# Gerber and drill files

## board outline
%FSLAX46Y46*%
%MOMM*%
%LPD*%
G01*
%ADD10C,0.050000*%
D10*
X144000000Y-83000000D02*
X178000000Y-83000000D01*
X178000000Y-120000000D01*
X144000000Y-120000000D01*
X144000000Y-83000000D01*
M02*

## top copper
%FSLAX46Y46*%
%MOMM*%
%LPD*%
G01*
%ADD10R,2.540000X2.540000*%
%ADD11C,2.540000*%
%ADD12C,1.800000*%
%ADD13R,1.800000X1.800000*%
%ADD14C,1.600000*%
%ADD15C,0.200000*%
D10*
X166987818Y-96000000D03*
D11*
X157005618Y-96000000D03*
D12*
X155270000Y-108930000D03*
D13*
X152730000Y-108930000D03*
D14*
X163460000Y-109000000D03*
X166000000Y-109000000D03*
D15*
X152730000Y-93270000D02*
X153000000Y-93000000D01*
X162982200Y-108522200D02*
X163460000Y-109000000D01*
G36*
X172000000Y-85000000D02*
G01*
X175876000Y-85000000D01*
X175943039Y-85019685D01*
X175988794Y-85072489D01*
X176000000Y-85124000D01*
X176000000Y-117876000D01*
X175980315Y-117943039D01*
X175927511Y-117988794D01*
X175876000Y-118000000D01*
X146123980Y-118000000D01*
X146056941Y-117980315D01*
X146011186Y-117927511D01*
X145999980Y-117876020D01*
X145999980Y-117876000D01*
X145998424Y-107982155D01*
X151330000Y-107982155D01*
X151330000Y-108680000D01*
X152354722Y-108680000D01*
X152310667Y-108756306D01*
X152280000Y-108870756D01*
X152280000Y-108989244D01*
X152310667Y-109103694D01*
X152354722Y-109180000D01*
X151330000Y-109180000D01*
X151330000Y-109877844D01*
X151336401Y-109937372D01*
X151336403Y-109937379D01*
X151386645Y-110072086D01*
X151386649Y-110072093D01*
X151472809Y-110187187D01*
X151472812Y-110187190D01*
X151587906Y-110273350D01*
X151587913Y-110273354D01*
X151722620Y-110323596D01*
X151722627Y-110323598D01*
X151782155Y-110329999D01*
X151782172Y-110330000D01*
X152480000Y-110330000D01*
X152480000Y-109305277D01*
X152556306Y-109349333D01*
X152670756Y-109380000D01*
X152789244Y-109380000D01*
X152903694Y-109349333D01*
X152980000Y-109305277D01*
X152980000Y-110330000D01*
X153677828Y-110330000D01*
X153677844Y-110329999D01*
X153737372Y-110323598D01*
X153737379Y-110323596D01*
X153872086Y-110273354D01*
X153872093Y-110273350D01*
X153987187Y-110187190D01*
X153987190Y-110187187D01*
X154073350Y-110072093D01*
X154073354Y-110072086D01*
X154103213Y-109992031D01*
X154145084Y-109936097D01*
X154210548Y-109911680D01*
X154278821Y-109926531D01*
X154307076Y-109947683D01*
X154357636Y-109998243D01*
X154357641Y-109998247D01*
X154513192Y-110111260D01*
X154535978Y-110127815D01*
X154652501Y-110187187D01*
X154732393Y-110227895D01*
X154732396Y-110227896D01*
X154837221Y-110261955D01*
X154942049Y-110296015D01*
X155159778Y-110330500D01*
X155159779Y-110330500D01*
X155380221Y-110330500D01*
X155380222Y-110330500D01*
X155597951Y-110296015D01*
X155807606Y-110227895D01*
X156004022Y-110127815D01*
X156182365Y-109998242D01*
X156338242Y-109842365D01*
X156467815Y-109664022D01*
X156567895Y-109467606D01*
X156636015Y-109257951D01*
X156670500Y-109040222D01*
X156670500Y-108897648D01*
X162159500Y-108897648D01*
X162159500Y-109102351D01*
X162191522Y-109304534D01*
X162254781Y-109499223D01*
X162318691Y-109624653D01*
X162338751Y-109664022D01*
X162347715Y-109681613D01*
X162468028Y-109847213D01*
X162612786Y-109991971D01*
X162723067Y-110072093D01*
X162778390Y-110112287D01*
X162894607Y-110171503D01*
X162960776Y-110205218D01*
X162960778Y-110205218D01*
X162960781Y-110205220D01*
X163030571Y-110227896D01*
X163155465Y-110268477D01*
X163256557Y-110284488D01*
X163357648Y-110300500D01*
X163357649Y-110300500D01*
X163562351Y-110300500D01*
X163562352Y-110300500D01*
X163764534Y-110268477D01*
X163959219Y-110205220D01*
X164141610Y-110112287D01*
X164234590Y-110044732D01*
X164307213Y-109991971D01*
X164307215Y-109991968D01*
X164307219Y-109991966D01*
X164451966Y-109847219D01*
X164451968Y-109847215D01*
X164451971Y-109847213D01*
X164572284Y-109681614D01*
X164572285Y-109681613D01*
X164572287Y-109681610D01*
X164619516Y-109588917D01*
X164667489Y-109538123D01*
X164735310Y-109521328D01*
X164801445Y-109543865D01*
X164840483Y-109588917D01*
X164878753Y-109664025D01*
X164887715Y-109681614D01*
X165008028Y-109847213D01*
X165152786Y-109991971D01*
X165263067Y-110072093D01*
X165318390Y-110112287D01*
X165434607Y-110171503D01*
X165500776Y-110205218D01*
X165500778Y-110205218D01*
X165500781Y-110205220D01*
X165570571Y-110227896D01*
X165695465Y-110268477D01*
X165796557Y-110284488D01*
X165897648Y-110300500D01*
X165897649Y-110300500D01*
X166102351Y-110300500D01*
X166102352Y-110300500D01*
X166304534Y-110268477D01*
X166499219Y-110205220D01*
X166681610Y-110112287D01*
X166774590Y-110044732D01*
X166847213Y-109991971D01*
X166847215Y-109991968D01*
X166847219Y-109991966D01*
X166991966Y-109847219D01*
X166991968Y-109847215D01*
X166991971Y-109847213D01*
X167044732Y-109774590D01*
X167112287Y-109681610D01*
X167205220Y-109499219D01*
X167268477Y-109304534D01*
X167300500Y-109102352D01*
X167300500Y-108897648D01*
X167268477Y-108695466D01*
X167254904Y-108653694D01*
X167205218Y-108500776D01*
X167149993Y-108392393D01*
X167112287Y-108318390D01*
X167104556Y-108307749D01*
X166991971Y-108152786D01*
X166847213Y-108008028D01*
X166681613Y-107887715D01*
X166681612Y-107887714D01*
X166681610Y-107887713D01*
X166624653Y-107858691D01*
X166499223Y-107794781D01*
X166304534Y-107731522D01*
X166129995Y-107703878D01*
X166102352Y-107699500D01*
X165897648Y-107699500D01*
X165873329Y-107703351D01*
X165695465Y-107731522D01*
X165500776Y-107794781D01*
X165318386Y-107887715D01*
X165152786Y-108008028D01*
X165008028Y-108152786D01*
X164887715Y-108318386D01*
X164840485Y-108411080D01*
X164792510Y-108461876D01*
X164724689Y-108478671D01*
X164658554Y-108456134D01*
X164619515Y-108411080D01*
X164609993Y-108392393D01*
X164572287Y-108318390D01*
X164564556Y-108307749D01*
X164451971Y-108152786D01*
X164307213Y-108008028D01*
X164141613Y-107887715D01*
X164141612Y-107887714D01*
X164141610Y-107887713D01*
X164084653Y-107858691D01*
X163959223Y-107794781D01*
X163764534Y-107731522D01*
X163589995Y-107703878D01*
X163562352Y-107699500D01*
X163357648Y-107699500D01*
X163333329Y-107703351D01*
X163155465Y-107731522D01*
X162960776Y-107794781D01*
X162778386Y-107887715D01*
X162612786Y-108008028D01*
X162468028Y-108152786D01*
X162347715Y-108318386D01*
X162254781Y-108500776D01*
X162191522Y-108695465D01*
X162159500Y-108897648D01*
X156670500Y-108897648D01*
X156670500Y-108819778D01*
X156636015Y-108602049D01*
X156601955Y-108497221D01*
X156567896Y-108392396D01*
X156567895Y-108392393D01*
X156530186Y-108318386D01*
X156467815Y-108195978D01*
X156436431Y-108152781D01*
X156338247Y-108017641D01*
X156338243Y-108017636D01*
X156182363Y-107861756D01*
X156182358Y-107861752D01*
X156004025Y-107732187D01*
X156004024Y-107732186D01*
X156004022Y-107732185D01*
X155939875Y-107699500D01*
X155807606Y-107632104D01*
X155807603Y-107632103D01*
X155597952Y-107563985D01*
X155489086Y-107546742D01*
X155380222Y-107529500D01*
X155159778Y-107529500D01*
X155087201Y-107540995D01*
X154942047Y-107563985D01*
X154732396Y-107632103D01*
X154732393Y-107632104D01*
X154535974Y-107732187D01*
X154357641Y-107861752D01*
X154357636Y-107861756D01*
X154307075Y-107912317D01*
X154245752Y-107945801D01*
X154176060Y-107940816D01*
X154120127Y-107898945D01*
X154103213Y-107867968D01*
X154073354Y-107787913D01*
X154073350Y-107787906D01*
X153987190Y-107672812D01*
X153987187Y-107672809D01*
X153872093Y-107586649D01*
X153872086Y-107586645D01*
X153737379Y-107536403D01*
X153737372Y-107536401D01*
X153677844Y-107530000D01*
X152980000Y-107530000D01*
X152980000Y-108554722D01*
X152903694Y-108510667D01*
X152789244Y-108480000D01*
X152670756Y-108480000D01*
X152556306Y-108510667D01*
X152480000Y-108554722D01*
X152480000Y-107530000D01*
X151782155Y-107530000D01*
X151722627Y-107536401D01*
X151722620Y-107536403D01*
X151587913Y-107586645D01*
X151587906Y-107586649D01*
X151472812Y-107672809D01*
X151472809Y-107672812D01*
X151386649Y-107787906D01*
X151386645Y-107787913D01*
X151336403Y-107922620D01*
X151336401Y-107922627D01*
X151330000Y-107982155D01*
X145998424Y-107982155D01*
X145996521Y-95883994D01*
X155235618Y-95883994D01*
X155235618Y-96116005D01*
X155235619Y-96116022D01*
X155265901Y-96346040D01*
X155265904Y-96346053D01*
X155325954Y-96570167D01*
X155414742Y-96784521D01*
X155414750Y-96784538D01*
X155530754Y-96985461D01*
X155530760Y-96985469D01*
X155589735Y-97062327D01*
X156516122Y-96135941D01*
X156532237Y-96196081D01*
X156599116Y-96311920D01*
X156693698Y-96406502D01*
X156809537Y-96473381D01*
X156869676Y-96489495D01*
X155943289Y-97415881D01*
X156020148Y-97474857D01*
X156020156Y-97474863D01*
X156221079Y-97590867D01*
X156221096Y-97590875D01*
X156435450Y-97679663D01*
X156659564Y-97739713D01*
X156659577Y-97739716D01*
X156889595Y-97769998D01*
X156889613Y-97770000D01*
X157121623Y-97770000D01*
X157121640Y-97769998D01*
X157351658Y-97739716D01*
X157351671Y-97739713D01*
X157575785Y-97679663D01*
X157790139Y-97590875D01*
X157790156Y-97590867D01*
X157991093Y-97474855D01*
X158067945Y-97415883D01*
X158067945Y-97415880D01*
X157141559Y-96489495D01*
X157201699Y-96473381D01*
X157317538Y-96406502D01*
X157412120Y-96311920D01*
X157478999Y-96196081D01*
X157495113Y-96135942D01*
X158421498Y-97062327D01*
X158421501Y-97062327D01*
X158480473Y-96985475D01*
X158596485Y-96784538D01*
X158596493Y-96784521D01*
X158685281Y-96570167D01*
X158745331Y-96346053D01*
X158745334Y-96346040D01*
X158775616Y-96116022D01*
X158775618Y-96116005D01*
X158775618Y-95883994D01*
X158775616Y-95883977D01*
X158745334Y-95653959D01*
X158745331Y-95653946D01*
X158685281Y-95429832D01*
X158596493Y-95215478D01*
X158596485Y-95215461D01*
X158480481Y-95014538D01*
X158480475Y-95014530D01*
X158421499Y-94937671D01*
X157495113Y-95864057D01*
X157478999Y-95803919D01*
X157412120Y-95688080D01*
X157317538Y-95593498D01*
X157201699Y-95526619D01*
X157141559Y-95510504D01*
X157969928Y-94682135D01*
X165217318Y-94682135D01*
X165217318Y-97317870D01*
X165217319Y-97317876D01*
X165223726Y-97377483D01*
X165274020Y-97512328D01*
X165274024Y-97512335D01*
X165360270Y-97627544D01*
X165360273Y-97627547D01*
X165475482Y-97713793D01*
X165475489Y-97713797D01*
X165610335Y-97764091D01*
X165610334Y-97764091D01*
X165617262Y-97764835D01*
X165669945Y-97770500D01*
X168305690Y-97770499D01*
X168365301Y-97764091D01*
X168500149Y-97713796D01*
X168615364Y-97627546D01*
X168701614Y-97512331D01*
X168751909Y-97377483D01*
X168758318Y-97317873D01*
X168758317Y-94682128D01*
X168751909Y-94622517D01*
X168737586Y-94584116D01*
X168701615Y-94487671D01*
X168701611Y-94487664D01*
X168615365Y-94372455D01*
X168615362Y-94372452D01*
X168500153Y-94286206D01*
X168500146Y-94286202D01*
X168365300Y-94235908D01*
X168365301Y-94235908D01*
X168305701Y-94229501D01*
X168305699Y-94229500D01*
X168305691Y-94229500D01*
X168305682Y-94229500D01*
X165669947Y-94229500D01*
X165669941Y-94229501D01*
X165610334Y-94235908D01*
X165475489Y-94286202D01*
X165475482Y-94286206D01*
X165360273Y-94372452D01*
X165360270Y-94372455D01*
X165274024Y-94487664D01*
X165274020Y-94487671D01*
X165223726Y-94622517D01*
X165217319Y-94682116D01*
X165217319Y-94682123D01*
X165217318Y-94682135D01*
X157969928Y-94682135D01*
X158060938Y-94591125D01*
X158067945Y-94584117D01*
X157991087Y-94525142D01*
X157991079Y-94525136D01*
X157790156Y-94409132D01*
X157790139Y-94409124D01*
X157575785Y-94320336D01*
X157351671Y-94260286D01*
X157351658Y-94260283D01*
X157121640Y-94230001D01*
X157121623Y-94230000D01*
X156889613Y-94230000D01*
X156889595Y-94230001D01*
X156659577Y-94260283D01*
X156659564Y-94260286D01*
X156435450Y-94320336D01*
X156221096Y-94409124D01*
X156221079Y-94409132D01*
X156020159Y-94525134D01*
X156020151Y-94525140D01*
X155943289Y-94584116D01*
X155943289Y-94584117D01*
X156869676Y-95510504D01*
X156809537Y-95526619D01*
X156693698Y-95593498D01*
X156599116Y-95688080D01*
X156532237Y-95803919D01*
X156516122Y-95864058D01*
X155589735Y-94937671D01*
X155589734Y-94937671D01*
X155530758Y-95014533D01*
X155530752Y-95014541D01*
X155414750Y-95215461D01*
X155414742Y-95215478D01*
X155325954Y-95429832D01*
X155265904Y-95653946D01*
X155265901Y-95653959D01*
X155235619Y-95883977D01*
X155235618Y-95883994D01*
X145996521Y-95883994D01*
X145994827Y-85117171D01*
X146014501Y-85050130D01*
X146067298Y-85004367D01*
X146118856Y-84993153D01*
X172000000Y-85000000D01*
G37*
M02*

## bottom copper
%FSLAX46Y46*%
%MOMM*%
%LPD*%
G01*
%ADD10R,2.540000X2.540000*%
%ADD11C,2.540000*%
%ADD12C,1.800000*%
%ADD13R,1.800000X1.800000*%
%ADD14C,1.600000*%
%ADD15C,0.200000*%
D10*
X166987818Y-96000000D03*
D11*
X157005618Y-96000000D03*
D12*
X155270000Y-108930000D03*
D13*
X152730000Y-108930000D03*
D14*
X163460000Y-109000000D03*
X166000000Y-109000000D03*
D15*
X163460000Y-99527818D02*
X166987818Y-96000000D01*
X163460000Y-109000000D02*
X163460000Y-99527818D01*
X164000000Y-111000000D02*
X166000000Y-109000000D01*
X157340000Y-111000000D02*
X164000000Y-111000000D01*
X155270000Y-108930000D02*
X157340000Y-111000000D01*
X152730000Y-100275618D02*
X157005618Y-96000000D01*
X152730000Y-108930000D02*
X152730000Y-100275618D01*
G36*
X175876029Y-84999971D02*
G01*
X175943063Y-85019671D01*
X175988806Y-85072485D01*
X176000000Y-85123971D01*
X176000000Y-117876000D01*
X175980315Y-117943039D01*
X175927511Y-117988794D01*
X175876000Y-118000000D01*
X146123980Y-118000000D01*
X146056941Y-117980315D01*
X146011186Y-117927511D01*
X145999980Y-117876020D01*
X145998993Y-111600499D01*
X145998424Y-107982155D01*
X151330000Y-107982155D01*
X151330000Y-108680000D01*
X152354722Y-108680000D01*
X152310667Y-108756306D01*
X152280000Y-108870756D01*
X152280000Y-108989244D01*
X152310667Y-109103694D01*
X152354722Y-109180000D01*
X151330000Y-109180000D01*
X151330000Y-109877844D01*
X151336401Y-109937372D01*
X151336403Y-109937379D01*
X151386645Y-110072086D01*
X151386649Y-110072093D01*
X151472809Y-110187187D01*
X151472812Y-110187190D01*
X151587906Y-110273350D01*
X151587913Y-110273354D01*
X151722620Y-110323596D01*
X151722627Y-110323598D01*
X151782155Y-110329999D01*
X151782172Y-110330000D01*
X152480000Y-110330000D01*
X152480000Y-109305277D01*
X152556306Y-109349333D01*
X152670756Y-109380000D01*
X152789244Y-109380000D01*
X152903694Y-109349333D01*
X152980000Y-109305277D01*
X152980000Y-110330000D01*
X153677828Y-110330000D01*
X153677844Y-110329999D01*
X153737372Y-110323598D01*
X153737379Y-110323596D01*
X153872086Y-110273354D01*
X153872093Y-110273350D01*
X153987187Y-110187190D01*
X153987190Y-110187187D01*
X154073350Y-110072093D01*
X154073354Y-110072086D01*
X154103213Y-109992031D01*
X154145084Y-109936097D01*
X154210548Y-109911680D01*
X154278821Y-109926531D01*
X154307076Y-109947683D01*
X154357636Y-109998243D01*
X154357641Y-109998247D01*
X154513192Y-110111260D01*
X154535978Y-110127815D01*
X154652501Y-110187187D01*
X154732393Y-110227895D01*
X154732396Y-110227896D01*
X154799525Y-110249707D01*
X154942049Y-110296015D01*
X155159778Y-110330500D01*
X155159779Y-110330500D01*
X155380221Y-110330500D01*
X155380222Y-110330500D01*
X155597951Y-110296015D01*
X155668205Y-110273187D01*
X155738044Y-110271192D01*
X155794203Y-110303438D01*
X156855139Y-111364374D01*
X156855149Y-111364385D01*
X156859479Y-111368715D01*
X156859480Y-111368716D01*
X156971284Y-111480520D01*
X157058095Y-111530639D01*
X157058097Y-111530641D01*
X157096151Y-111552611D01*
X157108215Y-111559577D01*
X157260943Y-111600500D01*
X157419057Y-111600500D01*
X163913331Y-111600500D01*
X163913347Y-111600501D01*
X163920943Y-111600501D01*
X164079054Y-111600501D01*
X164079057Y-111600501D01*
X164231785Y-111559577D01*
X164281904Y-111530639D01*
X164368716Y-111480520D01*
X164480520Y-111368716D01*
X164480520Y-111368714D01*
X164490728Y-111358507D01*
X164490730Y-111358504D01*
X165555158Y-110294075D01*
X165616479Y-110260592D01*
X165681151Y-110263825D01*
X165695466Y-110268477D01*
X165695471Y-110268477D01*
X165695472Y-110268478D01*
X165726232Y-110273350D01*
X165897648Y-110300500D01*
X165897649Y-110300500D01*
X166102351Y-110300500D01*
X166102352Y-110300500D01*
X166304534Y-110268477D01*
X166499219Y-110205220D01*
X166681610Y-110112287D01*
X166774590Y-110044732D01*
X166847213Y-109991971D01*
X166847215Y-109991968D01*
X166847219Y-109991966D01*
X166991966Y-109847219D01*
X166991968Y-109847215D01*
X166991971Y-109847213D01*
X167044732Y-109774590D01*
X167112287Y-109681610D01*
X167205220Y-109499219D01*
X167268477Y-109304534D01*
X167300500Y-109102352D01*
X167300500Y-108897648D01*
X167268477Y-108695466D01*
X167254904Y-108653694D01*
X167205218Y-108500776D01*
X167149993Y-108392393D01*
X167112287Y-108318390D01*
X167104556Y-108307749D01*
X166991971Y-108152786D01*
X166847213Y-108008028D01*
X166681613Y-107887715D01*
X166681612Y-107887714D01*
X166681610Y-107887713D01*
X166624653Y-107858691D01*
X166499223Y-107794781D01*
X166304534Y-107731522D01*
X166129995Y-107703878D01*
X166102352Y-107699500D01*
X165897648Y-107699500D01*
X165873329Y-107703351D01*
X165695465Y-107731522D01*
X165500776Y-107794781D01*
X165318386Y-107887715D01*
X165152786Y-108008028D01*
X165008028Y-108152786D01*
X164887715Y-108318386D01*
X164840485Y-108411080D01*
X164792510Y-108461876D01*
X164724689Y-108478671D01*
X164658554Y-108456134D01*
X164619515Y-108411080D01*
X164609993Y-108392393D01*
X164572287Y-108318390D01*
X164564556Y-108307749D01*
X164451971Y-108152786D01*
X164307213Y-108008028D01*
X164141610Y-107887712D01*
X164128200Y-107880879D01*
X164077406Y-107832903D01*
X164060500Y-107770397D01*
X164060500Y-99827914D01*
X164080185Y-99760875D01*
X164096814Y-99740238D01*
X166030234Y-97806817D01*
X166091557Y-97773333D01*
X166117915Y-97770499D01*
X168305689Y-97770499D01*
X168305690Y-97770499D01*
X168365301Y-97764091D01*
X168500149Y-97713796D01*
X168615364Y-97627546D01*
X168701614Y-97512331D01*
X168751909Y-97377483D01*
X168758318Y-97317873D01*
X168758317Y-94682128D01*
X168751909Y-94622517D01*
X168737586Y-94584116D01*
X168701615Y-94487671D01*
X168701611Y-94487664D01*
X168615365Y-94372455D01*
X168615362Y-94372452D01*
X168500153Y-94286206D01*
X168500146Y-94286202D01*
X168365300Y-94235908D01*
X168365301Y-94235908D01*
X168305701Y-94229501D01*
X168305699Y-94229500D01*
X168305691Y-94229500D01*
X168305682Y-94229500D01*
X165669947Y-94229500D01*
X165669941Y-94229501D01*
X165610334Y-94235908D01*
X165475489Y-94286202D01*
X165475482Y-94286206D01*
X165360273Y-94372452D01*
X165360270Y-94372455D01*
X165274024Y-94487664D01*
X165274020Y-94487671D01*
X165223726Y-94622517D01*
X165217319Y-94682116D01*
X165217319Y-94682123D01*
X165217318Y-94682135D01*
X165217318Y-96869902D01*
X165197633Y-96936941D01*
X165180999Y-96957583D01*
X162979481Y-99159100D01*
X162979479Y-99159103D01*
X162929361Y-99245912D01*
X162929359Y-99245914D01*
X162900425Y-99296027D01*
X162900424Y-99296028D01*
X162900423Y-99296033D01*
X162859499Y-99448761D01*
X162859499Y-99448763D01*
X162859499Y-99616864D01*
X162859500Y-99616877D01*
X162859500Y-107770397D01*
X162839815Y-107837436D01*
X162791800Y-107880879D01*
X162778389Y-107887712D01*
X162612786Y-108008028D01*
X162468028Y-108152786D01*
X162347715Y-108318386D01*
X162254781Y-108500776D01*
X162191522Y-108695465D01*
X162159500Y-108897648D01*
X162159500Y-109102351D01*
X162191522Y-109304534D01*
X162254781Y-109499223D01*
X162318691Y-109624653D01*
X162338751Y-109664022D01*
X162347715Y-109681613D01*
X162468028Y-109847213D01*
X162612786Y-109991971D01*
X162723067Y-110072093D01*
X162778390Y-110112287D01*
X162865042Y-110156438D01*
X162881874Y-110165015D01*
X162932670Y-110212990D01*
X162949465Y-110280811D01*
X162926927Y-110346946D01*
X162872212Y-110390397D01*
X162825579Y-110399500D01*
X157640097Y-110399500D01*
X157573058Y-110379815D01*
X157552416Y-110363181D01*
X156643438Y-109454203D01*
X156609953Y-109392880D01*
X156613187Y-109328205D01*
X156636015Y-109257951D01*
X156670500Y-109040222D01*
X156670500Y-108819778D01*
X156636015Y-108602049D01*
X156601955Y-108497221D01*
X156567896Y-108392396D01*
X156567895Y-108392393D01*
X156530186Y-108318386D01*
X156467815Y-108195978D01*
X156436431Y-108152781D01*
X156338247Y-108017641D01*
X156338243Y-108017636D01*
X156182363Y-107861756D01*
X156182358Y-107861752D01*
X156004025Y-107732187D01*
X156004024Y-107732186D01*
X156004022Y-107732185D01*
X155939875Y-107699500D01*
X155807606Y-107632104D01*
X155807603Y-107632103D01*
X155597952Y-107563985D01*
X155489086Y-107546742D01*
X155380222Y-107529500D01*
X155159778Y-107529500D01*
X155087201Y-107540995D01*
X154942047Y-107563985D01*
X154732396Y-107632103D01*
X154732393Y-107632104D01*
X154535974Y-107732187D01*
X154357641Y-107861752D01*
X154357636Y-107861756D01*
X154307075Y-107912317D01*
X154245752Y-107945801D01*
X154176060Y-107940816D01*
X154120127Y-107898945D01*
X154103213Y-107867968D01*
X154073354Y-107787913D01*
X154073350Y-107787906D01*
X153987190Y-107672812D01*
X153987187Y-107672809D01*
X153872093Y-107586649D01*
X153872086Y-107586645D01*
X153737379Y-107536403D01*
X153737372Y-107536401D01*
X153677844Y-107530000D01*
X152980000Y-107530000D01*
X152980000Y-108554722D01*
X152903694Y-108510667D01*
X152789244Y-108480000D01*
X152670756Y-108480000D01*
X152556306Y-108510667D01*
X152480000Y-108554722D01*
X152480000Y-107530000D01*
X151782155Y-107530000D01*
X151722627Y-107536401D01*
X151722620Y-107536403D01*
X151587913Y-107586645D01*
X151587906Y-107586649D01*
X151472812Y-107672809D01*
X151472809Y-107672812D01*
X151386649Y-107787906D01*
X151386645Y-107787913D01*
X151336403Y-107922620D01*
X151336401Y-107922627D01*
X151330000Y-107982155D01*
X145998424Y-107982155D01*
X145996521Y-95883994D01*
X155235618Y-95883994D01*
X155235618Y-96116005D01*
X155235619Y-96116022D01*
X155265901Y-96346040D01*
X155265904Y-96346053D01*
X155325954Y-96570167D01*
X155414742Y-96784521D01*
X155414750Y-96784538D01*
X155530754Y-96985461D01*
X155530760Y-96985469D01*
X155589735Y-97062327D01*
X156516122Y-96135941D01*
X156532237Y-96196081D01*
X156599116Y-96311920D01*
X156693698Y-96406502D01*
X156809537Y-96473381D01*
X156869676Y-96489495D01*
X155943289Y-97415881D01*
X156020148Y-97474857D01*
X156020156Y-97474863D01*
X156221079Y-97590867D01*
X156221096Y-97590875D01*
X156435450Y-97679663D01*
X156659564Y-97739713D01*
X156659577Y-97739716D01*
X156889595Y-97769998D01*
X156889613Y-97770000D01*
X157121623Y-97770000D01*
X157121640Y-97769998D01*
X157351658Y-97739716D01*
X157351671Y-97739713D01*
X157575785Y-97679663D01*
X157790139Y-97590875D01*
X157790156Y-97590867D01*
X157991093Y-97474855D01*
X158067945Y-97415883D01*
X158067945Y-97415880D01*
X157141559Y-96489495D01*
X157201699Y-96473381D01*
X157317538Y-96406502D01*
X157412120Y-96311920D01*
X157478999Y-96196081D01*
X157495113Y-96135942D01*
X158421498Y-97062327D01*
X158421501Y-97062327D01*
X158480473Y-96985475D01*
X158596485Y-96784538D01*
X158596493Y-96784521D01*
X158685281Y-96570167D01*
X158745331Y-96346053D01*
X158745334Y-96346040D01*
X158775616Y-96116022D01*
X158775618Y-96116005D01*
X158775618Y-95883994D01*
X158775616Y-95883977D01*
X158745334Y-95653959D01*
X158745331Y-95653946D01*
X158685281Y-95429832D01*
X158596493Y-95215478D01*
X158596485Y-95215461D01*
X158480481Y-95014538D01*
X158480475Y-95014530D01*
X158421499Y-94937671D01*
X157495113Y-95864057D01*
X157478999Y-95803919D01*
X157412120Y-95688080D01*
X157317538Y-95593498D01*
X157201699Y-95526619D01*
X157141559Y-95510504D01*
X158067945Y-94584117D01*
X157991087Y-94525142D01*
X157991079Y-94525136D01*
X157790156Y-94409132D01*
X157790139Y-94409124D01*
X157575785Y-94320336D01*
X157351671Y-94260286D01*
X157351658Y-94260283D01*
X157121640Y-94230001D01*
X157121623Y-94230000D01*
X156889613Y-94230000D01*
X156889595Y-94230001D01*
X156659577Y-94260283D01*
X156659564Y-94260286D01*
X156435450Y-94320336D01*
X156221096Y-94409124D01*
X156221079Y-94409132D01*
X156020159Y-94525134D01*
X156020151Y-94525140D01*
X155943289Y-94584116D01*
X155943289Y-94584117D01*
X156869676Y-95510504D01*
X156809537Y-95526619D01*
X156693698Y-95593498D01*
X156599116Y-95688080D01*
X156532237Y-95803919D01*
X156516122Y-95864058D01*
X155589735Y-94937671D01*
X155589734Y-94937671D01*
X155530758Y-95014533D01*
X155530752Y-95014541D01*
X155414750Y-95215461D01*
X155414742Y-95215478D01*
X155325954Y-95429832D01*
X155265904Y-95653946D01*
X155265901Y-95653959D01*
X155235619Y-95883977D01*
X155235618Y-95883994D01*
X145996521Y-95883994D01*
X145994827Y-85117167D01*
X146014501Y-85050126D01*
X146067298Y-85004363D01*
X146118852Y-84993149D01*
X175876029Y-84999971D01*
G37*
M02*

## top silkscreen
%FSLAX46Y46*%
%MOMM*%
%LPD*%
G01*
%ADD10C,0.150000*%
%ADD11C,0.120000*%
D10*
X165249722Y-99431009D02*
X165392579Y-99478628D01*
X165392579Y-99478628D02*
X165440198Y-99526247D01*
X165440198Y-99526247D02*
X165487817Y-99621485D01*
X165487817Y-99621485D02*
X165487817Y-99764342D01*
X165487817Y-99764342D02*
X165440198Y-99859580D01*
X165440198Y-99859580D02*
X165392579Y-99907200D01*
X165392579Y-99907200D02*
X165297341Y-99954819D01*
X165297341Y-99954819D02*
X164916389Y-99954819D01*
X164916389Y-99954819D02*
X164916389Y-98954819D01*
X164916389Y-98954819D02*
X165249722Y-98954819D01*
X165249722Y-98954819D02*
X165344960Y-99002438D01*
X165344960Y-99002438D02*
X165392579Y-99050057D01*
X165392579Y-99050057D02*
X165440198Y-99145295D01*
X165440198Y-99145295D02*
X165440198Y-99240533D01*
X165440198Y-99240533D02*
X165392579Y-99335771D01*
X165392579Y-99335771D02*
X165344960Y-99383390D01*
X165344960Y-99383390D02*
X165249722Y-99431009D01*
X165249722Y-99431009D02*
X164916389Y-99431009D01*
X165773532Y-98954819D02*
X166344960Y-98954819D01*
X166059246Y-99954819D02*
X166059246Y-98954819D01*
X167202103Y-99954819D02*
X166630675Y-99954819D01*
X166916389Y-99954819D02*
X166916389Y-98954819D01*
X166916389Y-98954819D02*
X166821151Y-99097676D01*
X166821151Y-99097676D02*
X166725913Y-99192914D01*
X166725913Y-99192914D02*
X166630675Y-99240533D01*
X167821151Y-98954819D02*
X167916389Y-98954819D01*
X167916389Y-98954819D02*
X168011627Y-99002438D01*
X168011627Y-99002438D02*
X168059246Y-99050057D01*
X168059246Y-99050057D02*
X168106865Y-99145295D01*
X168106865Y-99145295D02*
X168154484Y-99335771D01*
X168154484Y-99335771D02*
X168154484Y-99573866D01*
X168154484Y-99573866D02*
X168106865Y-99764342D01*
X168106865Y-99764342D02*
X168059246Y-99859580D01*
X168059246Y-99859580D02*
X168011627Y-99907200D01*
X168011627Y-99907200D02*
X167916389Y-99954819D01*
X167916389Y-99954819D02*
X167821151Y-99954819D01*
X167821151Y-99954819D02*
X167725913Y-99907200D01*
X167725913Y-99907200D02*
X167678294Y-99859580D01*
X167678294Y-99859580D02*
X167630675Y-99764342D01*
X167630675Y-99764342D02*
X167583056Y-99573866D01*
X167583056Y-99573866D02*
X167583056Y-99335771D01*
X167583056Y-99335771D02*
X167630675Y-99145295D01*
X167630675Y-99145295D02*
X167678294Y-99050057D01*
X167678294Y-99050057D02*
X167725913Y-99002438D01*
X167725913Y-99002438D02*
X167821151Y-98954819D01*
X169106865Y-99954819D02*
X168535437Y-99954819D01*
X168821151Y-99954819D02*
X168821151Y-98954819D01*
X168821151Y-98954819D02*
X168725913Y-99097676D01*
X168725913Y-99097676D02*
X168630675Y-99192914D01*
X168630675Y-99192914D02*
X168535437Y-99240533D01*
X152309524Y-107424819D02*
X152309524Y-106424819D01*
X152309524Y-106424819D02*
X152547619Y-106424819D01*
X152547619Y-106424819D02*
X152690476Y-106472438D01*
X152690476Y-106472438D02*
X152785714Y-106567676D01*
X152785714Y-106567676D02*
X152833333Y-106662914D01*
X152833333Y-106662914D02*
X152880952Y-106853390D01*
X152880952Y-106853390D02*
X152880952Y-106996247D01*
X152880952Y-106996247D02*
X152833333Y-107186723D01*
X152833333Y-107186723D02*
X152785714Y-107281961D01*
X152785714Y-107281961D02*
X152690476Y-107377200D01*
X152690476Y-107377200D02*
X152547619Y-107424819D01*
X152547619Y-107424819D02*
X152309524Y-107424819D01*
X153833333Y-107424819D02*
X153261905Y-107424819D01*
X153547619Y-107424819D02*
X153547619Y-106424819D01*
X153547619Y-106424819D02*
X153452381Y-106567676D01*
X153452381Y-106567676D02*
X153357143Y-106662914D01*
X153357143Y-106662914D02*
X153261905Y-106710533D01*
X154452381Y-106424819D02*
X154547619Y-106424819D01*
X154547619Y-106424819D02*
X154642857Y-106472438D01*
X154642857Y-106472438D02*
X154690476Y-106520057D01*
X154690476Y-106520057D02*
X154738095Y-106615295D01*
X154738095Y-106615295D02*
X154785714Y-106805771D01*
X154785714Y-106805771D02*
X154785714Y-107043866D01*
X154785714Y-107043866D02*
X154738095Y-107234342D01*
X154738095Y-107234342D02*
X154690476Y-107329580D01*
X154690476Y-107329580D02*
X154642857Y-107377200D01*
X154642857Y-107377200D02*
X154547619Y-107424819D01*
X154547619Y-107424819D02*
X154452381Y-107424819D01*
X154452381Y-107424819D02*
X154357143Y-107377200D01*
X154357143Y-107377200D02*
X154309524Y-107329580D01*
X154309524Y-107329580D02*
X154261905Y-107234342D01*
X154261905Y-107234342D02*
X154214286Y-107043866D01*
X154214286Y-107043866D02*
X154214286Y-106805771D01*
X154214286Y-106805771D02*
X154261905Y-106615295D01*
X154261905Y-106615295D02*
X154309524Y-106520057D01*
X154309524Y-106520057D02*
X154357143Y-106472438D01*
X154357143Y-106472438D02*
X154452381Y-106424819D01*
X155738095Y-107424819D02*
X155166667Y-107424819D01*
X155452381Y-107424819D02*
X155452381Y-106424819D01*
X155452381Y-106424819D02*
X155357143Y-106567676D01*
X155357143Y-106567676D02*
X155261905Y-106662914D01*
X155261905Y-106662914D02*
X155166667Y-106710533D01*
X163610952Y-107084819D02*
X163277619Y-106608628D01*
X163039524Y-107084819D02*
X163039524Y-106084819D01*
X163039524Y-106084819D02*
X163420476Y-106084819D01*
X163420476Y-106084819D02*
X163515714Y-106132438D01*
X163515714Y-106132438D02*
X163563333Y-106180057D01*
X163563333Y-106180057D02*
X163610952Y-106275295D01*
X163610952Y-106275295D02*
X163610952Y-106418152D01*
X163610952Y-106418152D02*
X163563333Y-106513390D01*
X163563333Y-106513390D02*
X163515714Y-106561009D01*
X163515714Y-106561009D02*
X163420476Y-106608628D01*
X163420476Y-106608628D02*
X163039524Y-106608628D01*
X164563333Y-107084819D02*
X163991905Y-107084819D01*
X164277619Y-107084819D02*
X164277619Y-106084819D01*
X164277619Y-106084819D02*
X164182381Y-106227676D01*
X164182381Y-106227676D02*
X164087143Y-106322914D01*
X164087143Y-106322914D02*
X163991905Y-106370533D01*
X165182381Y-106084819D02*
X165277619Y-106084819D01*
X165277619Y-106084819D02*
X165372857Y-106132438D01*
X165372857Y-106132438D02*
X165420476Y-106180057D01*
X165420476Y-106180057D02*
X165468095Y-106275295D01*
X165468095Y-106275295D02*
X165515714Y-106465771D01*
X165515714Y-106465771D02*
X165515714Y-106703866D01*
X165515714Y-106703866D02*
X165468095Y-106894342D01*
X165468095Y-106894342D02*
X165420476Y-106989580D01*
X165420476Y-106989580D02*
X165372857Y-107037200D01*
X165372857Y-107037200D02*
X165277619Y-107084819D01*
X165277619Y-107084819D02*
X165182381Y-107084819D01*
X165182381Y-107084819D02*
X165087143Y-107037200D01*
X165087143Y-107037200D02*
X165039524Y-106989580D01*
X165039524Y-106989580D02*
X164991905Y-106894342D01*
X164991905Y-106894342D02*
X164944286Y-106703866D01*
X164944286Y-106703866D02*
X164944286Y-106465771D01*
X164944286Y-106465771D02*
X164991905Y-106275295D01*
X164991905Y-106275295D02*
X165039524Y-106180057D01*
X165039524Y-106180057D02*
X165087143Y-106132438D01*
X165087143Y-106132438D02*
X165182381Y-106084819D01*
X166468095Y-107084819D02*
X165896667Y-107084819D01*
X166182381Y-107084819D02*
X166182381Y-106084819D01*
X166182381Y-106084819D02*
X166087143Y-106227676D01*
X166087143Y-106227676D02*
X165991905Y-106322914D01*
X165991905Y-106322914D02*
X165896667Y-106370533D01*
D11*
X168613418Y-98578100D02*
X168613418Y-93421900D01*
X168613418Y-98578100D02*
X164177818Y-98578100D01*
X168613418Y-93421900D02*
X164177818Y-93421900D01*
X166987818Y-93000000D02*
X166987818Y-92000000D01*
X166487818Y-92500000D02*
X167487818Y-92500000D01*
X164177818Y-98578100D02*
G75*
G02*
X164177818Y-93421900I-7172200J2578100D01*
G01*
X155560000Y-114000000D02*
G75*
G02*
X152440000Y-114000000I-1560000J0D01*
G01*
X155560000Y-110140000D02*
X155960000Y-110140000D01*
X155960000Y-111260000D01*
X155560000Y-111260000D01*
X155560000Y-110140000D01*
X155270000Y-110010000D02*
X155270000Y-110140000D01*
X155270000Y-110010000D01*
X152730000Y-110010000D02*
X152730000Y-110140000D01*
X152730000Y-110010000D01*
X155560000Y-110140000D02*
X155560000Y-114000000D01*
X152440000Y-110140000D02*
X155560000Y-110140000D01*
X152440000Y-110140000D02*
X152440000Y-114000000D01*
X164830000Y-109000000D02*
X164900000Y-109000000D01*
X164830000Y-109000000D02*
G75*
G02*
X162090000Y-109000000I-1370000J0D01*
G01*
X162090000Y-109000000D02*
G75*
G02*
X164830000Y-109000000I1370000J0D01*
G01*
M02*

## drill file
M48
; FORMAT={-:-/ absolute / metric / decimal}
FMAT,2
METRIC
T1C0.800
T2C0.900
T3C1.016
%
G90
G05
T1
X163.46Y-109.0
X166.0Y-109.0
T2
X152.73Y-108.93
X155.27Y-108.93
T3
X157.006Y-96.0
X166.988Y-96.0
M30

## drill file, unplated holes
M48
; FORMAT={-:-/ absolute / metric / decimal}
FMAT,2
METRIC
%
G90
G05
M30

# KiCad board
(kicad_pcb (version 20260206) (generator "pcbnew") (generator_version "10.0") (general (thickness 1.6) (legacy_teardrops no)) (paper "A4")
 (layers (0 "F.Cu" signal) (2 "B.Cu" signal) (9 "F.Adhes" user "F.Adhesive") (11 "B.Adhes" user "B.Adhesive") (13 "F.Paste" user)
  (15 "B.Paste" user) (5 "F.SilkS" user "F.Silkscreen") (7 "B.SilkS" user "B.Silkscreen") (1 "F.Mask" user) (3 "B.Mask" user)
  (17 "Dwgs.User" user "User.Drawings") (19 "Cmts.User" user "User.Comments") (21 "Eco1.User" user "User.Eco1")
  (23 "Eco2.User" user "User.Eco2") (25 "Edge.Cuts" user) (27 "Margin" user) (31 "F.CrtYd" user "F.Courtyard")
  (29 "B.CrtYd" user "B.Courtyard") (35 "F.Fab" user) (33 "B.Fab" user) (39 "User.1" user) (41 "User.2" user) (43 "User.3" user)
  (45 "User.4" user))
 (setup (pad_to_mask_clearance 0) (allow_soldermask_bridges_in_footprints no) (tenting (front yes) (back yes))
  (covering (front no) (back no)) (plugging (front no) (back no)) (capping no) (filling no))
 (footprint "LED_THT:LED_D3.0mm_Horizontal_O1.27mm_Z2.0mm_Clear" (layer "F.Cu") (at 152.73 108.93)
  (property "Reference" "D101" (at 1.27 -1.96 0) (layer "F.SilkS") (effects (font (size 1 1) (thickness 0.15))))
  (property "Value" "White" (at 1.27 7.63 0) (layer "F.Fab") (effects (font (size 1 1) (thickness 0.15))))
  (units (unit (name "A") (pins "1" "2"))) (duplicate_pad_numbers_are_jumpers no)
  (fp_line (start -0.29 1.21) (end -0.29 5.07) (stroke (width 0.12) (type solid)) (layer "F.SilkS"))
  (fp_line (start -0.29 1.21) (end 2.83 1.21) (stroke (width 0.12) (type solid)) (layer "F.SilkS"))
  (fp_line (start 2.83 1.21) (end 2.83 5.07) (stroke (width 0.12) (type solid)) (layer "F.SilkS"))
  (fp_rect (start 0 1.08) (end 0 1.21) (stroke (width 0.12) (type solid)) (fill no) (layer "F.SilkS"))
  (fp_rect (start 2.54 1.08) (end 2.54 1.21) (stroke (width 0.12) (type solid)) (fill no) (layer "F.SilkS"))
  (fp_rect (start 2.83 1.21) (end 3.23 2.33) (stroke (width 0.12) (type solid)) (fill no) (layer "F.SilkS"))
  (fp_arc (start 2.83 5.07) (mid 1.27 6.63) (end -0.29 5.07) (stroke (width 0.12) (type solid)) (layer "F.SilkS"))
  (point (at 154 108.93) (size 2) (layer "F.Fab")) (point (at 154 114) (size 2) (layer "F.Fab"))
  (pad "1" thru_hole rect (at 0 0) (size 1.8 1.8) (drill 0.9) (layers "*.Cu" "*.Mask") (remove_unused_layers no) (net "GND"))
  (pad "2" thru_hole circle (at 2.54 0) (size 1.8 1.8) (drill 0.9) (layers "*.Cu" "*.Mask") (remove_unused_layers no) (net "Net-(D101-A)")))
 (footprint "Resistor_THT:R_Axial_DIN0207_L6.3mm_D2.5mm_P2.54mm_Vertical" (layer "F.Cu") (at 163.46 109)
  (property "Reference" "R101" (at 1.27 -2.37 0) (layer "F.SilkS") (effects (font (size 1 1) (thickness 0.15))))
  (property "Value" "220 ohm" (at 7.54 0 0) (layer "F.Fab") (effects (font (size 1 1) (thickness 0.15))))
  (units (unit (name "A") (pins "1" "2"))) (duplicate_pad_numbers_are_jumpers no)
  (fp_line (start 1.37 0) (end 1.44 0) (stroke (width 0.12) (type solid)) (layer "F.SilkS"))
  (fp_circle (center 0 0) (end 1.37 0) (stroke (width 0.12) (type solid)) (fill no) (layer "F.SilkS"))
  (pad "1" thru_hole circle (at 0 0) (size 1.6 1.6) (drill 0.8) (layers "*.Cu" "*.Mask") (remove_unused_layers no) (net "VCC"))
  (pad "2" thru_hole circle (at 2.54 0) (size 1.6 1.6) (drill 0.8) (layers "*.Cu" "*.Mask") (remove_unused_layers no) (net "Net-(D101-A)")))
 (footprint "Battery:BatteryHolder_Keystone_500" (layer "F.Cu") (at 166.987818 96 180)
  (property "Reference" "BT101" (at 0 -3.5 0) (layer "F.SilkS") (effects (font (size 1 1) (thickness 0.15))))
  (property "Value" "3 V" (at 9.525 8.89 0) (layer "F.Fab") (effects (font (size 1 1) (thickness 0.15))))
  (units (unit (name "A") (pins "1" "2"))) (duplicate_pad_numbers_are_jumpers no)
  (fp_line (start 0.5 3.5) (end -0.5 3.5) (stroke (width 0.12) (type default)) (layer "F.SilkS"))
  (fp_line (start 0 3) (end 0 4) (stroke (width 0.12) (type default)) (layer "F.SilkS"))
  (fp_line (start -1.6256 2.5781) (end 2.81 2.5781) (stroke (width 0.12) (type solid)) (layer "F.SilkS"))
  (fp_line (start -1.6256 -2.5781) (end 2.81 -2.5781) (stroke (width 0.12) (type solid)) (layer "F.SilkS"))
  (fp_line (start -1.6256 -2.5781) (end -1.6256 2.5781) (stroke (width 0.12) (type default)) (layer "F.SilkS"))
  (fp_arc (start 2.81 -2.5781) (mid 17.603686 0) (end 2.81 2.5781) (stroke (width 0.12) (type default)) (layer "F.SilkS"))
  (pad "1" thru_hole rect (at 0 0 180) (size 2.54 2.54) (drill 1.016) (layers "*.Cu" "*.Mask") (remove_unused_layers no) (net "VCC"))
  (pad "2" thru_hole circle (at 9.9822 0 180) (size 2.54 2.54) (drill 1.016) (layers "*.Cu" "*.Mask") (remove_unused_layers no) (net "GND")))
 (gr_rect (start 144 83) (end 178 120) (stroke (width 0.05) (type default)) (fill no) (layer "Edge.Cuts"))
 (segment (start 152.73 93.27) (end 153 93) (width 0.2) (layer "F.Cu") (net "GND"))
 (segment (start 152.73 108.93) (end 152.73 100.275618) (width 0.2) (layer "B.Cu") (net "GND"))
 (segment (start 152.73 100.275618) (end 157.005618 96) (width 0.2) (layer "B.Cu") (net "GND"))
 (segment (start 162.9822 108.5222) (end 163.46 109) (width 0.2) (layer "F.Cu") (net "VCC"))
 (segment (start 163.46 109) (end 163.46 99.527818) (width 0.2) (layer "B.Cu") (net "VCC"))
 (segment (start 163.46 99.527818) (end 166.987818 96) (width 0.2) (layer "B.Cu") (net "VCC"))
 (segment (start 157.34 111) (end 164 111) (width 0.2) (layer "B.Cu") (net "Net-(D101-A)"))
 (segment (start 155.27 108.93) (end 157.34 111) (width 0.2) (layer "B.Cu") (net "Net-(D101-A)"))
 (segment (start 164 111) (end 166 109) (width 0.2) (layer "B.Cu") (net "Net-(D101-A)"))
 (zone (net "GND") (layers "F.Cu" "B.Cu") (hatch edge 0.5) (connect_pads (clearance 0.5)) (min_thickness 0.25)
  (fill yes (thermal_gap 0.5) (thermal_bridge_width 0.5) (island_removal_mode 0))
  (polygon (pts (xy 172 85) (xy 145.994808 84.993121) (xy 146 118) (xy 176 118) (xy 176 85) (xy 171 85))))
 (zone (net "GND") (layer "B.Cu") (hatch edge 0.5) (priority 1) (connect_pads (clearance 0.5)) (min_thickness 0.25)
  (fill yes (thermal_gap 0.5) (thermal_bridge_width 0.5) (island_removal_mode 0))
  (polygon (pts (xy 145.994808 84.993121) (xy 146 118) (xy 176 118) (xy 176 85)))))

